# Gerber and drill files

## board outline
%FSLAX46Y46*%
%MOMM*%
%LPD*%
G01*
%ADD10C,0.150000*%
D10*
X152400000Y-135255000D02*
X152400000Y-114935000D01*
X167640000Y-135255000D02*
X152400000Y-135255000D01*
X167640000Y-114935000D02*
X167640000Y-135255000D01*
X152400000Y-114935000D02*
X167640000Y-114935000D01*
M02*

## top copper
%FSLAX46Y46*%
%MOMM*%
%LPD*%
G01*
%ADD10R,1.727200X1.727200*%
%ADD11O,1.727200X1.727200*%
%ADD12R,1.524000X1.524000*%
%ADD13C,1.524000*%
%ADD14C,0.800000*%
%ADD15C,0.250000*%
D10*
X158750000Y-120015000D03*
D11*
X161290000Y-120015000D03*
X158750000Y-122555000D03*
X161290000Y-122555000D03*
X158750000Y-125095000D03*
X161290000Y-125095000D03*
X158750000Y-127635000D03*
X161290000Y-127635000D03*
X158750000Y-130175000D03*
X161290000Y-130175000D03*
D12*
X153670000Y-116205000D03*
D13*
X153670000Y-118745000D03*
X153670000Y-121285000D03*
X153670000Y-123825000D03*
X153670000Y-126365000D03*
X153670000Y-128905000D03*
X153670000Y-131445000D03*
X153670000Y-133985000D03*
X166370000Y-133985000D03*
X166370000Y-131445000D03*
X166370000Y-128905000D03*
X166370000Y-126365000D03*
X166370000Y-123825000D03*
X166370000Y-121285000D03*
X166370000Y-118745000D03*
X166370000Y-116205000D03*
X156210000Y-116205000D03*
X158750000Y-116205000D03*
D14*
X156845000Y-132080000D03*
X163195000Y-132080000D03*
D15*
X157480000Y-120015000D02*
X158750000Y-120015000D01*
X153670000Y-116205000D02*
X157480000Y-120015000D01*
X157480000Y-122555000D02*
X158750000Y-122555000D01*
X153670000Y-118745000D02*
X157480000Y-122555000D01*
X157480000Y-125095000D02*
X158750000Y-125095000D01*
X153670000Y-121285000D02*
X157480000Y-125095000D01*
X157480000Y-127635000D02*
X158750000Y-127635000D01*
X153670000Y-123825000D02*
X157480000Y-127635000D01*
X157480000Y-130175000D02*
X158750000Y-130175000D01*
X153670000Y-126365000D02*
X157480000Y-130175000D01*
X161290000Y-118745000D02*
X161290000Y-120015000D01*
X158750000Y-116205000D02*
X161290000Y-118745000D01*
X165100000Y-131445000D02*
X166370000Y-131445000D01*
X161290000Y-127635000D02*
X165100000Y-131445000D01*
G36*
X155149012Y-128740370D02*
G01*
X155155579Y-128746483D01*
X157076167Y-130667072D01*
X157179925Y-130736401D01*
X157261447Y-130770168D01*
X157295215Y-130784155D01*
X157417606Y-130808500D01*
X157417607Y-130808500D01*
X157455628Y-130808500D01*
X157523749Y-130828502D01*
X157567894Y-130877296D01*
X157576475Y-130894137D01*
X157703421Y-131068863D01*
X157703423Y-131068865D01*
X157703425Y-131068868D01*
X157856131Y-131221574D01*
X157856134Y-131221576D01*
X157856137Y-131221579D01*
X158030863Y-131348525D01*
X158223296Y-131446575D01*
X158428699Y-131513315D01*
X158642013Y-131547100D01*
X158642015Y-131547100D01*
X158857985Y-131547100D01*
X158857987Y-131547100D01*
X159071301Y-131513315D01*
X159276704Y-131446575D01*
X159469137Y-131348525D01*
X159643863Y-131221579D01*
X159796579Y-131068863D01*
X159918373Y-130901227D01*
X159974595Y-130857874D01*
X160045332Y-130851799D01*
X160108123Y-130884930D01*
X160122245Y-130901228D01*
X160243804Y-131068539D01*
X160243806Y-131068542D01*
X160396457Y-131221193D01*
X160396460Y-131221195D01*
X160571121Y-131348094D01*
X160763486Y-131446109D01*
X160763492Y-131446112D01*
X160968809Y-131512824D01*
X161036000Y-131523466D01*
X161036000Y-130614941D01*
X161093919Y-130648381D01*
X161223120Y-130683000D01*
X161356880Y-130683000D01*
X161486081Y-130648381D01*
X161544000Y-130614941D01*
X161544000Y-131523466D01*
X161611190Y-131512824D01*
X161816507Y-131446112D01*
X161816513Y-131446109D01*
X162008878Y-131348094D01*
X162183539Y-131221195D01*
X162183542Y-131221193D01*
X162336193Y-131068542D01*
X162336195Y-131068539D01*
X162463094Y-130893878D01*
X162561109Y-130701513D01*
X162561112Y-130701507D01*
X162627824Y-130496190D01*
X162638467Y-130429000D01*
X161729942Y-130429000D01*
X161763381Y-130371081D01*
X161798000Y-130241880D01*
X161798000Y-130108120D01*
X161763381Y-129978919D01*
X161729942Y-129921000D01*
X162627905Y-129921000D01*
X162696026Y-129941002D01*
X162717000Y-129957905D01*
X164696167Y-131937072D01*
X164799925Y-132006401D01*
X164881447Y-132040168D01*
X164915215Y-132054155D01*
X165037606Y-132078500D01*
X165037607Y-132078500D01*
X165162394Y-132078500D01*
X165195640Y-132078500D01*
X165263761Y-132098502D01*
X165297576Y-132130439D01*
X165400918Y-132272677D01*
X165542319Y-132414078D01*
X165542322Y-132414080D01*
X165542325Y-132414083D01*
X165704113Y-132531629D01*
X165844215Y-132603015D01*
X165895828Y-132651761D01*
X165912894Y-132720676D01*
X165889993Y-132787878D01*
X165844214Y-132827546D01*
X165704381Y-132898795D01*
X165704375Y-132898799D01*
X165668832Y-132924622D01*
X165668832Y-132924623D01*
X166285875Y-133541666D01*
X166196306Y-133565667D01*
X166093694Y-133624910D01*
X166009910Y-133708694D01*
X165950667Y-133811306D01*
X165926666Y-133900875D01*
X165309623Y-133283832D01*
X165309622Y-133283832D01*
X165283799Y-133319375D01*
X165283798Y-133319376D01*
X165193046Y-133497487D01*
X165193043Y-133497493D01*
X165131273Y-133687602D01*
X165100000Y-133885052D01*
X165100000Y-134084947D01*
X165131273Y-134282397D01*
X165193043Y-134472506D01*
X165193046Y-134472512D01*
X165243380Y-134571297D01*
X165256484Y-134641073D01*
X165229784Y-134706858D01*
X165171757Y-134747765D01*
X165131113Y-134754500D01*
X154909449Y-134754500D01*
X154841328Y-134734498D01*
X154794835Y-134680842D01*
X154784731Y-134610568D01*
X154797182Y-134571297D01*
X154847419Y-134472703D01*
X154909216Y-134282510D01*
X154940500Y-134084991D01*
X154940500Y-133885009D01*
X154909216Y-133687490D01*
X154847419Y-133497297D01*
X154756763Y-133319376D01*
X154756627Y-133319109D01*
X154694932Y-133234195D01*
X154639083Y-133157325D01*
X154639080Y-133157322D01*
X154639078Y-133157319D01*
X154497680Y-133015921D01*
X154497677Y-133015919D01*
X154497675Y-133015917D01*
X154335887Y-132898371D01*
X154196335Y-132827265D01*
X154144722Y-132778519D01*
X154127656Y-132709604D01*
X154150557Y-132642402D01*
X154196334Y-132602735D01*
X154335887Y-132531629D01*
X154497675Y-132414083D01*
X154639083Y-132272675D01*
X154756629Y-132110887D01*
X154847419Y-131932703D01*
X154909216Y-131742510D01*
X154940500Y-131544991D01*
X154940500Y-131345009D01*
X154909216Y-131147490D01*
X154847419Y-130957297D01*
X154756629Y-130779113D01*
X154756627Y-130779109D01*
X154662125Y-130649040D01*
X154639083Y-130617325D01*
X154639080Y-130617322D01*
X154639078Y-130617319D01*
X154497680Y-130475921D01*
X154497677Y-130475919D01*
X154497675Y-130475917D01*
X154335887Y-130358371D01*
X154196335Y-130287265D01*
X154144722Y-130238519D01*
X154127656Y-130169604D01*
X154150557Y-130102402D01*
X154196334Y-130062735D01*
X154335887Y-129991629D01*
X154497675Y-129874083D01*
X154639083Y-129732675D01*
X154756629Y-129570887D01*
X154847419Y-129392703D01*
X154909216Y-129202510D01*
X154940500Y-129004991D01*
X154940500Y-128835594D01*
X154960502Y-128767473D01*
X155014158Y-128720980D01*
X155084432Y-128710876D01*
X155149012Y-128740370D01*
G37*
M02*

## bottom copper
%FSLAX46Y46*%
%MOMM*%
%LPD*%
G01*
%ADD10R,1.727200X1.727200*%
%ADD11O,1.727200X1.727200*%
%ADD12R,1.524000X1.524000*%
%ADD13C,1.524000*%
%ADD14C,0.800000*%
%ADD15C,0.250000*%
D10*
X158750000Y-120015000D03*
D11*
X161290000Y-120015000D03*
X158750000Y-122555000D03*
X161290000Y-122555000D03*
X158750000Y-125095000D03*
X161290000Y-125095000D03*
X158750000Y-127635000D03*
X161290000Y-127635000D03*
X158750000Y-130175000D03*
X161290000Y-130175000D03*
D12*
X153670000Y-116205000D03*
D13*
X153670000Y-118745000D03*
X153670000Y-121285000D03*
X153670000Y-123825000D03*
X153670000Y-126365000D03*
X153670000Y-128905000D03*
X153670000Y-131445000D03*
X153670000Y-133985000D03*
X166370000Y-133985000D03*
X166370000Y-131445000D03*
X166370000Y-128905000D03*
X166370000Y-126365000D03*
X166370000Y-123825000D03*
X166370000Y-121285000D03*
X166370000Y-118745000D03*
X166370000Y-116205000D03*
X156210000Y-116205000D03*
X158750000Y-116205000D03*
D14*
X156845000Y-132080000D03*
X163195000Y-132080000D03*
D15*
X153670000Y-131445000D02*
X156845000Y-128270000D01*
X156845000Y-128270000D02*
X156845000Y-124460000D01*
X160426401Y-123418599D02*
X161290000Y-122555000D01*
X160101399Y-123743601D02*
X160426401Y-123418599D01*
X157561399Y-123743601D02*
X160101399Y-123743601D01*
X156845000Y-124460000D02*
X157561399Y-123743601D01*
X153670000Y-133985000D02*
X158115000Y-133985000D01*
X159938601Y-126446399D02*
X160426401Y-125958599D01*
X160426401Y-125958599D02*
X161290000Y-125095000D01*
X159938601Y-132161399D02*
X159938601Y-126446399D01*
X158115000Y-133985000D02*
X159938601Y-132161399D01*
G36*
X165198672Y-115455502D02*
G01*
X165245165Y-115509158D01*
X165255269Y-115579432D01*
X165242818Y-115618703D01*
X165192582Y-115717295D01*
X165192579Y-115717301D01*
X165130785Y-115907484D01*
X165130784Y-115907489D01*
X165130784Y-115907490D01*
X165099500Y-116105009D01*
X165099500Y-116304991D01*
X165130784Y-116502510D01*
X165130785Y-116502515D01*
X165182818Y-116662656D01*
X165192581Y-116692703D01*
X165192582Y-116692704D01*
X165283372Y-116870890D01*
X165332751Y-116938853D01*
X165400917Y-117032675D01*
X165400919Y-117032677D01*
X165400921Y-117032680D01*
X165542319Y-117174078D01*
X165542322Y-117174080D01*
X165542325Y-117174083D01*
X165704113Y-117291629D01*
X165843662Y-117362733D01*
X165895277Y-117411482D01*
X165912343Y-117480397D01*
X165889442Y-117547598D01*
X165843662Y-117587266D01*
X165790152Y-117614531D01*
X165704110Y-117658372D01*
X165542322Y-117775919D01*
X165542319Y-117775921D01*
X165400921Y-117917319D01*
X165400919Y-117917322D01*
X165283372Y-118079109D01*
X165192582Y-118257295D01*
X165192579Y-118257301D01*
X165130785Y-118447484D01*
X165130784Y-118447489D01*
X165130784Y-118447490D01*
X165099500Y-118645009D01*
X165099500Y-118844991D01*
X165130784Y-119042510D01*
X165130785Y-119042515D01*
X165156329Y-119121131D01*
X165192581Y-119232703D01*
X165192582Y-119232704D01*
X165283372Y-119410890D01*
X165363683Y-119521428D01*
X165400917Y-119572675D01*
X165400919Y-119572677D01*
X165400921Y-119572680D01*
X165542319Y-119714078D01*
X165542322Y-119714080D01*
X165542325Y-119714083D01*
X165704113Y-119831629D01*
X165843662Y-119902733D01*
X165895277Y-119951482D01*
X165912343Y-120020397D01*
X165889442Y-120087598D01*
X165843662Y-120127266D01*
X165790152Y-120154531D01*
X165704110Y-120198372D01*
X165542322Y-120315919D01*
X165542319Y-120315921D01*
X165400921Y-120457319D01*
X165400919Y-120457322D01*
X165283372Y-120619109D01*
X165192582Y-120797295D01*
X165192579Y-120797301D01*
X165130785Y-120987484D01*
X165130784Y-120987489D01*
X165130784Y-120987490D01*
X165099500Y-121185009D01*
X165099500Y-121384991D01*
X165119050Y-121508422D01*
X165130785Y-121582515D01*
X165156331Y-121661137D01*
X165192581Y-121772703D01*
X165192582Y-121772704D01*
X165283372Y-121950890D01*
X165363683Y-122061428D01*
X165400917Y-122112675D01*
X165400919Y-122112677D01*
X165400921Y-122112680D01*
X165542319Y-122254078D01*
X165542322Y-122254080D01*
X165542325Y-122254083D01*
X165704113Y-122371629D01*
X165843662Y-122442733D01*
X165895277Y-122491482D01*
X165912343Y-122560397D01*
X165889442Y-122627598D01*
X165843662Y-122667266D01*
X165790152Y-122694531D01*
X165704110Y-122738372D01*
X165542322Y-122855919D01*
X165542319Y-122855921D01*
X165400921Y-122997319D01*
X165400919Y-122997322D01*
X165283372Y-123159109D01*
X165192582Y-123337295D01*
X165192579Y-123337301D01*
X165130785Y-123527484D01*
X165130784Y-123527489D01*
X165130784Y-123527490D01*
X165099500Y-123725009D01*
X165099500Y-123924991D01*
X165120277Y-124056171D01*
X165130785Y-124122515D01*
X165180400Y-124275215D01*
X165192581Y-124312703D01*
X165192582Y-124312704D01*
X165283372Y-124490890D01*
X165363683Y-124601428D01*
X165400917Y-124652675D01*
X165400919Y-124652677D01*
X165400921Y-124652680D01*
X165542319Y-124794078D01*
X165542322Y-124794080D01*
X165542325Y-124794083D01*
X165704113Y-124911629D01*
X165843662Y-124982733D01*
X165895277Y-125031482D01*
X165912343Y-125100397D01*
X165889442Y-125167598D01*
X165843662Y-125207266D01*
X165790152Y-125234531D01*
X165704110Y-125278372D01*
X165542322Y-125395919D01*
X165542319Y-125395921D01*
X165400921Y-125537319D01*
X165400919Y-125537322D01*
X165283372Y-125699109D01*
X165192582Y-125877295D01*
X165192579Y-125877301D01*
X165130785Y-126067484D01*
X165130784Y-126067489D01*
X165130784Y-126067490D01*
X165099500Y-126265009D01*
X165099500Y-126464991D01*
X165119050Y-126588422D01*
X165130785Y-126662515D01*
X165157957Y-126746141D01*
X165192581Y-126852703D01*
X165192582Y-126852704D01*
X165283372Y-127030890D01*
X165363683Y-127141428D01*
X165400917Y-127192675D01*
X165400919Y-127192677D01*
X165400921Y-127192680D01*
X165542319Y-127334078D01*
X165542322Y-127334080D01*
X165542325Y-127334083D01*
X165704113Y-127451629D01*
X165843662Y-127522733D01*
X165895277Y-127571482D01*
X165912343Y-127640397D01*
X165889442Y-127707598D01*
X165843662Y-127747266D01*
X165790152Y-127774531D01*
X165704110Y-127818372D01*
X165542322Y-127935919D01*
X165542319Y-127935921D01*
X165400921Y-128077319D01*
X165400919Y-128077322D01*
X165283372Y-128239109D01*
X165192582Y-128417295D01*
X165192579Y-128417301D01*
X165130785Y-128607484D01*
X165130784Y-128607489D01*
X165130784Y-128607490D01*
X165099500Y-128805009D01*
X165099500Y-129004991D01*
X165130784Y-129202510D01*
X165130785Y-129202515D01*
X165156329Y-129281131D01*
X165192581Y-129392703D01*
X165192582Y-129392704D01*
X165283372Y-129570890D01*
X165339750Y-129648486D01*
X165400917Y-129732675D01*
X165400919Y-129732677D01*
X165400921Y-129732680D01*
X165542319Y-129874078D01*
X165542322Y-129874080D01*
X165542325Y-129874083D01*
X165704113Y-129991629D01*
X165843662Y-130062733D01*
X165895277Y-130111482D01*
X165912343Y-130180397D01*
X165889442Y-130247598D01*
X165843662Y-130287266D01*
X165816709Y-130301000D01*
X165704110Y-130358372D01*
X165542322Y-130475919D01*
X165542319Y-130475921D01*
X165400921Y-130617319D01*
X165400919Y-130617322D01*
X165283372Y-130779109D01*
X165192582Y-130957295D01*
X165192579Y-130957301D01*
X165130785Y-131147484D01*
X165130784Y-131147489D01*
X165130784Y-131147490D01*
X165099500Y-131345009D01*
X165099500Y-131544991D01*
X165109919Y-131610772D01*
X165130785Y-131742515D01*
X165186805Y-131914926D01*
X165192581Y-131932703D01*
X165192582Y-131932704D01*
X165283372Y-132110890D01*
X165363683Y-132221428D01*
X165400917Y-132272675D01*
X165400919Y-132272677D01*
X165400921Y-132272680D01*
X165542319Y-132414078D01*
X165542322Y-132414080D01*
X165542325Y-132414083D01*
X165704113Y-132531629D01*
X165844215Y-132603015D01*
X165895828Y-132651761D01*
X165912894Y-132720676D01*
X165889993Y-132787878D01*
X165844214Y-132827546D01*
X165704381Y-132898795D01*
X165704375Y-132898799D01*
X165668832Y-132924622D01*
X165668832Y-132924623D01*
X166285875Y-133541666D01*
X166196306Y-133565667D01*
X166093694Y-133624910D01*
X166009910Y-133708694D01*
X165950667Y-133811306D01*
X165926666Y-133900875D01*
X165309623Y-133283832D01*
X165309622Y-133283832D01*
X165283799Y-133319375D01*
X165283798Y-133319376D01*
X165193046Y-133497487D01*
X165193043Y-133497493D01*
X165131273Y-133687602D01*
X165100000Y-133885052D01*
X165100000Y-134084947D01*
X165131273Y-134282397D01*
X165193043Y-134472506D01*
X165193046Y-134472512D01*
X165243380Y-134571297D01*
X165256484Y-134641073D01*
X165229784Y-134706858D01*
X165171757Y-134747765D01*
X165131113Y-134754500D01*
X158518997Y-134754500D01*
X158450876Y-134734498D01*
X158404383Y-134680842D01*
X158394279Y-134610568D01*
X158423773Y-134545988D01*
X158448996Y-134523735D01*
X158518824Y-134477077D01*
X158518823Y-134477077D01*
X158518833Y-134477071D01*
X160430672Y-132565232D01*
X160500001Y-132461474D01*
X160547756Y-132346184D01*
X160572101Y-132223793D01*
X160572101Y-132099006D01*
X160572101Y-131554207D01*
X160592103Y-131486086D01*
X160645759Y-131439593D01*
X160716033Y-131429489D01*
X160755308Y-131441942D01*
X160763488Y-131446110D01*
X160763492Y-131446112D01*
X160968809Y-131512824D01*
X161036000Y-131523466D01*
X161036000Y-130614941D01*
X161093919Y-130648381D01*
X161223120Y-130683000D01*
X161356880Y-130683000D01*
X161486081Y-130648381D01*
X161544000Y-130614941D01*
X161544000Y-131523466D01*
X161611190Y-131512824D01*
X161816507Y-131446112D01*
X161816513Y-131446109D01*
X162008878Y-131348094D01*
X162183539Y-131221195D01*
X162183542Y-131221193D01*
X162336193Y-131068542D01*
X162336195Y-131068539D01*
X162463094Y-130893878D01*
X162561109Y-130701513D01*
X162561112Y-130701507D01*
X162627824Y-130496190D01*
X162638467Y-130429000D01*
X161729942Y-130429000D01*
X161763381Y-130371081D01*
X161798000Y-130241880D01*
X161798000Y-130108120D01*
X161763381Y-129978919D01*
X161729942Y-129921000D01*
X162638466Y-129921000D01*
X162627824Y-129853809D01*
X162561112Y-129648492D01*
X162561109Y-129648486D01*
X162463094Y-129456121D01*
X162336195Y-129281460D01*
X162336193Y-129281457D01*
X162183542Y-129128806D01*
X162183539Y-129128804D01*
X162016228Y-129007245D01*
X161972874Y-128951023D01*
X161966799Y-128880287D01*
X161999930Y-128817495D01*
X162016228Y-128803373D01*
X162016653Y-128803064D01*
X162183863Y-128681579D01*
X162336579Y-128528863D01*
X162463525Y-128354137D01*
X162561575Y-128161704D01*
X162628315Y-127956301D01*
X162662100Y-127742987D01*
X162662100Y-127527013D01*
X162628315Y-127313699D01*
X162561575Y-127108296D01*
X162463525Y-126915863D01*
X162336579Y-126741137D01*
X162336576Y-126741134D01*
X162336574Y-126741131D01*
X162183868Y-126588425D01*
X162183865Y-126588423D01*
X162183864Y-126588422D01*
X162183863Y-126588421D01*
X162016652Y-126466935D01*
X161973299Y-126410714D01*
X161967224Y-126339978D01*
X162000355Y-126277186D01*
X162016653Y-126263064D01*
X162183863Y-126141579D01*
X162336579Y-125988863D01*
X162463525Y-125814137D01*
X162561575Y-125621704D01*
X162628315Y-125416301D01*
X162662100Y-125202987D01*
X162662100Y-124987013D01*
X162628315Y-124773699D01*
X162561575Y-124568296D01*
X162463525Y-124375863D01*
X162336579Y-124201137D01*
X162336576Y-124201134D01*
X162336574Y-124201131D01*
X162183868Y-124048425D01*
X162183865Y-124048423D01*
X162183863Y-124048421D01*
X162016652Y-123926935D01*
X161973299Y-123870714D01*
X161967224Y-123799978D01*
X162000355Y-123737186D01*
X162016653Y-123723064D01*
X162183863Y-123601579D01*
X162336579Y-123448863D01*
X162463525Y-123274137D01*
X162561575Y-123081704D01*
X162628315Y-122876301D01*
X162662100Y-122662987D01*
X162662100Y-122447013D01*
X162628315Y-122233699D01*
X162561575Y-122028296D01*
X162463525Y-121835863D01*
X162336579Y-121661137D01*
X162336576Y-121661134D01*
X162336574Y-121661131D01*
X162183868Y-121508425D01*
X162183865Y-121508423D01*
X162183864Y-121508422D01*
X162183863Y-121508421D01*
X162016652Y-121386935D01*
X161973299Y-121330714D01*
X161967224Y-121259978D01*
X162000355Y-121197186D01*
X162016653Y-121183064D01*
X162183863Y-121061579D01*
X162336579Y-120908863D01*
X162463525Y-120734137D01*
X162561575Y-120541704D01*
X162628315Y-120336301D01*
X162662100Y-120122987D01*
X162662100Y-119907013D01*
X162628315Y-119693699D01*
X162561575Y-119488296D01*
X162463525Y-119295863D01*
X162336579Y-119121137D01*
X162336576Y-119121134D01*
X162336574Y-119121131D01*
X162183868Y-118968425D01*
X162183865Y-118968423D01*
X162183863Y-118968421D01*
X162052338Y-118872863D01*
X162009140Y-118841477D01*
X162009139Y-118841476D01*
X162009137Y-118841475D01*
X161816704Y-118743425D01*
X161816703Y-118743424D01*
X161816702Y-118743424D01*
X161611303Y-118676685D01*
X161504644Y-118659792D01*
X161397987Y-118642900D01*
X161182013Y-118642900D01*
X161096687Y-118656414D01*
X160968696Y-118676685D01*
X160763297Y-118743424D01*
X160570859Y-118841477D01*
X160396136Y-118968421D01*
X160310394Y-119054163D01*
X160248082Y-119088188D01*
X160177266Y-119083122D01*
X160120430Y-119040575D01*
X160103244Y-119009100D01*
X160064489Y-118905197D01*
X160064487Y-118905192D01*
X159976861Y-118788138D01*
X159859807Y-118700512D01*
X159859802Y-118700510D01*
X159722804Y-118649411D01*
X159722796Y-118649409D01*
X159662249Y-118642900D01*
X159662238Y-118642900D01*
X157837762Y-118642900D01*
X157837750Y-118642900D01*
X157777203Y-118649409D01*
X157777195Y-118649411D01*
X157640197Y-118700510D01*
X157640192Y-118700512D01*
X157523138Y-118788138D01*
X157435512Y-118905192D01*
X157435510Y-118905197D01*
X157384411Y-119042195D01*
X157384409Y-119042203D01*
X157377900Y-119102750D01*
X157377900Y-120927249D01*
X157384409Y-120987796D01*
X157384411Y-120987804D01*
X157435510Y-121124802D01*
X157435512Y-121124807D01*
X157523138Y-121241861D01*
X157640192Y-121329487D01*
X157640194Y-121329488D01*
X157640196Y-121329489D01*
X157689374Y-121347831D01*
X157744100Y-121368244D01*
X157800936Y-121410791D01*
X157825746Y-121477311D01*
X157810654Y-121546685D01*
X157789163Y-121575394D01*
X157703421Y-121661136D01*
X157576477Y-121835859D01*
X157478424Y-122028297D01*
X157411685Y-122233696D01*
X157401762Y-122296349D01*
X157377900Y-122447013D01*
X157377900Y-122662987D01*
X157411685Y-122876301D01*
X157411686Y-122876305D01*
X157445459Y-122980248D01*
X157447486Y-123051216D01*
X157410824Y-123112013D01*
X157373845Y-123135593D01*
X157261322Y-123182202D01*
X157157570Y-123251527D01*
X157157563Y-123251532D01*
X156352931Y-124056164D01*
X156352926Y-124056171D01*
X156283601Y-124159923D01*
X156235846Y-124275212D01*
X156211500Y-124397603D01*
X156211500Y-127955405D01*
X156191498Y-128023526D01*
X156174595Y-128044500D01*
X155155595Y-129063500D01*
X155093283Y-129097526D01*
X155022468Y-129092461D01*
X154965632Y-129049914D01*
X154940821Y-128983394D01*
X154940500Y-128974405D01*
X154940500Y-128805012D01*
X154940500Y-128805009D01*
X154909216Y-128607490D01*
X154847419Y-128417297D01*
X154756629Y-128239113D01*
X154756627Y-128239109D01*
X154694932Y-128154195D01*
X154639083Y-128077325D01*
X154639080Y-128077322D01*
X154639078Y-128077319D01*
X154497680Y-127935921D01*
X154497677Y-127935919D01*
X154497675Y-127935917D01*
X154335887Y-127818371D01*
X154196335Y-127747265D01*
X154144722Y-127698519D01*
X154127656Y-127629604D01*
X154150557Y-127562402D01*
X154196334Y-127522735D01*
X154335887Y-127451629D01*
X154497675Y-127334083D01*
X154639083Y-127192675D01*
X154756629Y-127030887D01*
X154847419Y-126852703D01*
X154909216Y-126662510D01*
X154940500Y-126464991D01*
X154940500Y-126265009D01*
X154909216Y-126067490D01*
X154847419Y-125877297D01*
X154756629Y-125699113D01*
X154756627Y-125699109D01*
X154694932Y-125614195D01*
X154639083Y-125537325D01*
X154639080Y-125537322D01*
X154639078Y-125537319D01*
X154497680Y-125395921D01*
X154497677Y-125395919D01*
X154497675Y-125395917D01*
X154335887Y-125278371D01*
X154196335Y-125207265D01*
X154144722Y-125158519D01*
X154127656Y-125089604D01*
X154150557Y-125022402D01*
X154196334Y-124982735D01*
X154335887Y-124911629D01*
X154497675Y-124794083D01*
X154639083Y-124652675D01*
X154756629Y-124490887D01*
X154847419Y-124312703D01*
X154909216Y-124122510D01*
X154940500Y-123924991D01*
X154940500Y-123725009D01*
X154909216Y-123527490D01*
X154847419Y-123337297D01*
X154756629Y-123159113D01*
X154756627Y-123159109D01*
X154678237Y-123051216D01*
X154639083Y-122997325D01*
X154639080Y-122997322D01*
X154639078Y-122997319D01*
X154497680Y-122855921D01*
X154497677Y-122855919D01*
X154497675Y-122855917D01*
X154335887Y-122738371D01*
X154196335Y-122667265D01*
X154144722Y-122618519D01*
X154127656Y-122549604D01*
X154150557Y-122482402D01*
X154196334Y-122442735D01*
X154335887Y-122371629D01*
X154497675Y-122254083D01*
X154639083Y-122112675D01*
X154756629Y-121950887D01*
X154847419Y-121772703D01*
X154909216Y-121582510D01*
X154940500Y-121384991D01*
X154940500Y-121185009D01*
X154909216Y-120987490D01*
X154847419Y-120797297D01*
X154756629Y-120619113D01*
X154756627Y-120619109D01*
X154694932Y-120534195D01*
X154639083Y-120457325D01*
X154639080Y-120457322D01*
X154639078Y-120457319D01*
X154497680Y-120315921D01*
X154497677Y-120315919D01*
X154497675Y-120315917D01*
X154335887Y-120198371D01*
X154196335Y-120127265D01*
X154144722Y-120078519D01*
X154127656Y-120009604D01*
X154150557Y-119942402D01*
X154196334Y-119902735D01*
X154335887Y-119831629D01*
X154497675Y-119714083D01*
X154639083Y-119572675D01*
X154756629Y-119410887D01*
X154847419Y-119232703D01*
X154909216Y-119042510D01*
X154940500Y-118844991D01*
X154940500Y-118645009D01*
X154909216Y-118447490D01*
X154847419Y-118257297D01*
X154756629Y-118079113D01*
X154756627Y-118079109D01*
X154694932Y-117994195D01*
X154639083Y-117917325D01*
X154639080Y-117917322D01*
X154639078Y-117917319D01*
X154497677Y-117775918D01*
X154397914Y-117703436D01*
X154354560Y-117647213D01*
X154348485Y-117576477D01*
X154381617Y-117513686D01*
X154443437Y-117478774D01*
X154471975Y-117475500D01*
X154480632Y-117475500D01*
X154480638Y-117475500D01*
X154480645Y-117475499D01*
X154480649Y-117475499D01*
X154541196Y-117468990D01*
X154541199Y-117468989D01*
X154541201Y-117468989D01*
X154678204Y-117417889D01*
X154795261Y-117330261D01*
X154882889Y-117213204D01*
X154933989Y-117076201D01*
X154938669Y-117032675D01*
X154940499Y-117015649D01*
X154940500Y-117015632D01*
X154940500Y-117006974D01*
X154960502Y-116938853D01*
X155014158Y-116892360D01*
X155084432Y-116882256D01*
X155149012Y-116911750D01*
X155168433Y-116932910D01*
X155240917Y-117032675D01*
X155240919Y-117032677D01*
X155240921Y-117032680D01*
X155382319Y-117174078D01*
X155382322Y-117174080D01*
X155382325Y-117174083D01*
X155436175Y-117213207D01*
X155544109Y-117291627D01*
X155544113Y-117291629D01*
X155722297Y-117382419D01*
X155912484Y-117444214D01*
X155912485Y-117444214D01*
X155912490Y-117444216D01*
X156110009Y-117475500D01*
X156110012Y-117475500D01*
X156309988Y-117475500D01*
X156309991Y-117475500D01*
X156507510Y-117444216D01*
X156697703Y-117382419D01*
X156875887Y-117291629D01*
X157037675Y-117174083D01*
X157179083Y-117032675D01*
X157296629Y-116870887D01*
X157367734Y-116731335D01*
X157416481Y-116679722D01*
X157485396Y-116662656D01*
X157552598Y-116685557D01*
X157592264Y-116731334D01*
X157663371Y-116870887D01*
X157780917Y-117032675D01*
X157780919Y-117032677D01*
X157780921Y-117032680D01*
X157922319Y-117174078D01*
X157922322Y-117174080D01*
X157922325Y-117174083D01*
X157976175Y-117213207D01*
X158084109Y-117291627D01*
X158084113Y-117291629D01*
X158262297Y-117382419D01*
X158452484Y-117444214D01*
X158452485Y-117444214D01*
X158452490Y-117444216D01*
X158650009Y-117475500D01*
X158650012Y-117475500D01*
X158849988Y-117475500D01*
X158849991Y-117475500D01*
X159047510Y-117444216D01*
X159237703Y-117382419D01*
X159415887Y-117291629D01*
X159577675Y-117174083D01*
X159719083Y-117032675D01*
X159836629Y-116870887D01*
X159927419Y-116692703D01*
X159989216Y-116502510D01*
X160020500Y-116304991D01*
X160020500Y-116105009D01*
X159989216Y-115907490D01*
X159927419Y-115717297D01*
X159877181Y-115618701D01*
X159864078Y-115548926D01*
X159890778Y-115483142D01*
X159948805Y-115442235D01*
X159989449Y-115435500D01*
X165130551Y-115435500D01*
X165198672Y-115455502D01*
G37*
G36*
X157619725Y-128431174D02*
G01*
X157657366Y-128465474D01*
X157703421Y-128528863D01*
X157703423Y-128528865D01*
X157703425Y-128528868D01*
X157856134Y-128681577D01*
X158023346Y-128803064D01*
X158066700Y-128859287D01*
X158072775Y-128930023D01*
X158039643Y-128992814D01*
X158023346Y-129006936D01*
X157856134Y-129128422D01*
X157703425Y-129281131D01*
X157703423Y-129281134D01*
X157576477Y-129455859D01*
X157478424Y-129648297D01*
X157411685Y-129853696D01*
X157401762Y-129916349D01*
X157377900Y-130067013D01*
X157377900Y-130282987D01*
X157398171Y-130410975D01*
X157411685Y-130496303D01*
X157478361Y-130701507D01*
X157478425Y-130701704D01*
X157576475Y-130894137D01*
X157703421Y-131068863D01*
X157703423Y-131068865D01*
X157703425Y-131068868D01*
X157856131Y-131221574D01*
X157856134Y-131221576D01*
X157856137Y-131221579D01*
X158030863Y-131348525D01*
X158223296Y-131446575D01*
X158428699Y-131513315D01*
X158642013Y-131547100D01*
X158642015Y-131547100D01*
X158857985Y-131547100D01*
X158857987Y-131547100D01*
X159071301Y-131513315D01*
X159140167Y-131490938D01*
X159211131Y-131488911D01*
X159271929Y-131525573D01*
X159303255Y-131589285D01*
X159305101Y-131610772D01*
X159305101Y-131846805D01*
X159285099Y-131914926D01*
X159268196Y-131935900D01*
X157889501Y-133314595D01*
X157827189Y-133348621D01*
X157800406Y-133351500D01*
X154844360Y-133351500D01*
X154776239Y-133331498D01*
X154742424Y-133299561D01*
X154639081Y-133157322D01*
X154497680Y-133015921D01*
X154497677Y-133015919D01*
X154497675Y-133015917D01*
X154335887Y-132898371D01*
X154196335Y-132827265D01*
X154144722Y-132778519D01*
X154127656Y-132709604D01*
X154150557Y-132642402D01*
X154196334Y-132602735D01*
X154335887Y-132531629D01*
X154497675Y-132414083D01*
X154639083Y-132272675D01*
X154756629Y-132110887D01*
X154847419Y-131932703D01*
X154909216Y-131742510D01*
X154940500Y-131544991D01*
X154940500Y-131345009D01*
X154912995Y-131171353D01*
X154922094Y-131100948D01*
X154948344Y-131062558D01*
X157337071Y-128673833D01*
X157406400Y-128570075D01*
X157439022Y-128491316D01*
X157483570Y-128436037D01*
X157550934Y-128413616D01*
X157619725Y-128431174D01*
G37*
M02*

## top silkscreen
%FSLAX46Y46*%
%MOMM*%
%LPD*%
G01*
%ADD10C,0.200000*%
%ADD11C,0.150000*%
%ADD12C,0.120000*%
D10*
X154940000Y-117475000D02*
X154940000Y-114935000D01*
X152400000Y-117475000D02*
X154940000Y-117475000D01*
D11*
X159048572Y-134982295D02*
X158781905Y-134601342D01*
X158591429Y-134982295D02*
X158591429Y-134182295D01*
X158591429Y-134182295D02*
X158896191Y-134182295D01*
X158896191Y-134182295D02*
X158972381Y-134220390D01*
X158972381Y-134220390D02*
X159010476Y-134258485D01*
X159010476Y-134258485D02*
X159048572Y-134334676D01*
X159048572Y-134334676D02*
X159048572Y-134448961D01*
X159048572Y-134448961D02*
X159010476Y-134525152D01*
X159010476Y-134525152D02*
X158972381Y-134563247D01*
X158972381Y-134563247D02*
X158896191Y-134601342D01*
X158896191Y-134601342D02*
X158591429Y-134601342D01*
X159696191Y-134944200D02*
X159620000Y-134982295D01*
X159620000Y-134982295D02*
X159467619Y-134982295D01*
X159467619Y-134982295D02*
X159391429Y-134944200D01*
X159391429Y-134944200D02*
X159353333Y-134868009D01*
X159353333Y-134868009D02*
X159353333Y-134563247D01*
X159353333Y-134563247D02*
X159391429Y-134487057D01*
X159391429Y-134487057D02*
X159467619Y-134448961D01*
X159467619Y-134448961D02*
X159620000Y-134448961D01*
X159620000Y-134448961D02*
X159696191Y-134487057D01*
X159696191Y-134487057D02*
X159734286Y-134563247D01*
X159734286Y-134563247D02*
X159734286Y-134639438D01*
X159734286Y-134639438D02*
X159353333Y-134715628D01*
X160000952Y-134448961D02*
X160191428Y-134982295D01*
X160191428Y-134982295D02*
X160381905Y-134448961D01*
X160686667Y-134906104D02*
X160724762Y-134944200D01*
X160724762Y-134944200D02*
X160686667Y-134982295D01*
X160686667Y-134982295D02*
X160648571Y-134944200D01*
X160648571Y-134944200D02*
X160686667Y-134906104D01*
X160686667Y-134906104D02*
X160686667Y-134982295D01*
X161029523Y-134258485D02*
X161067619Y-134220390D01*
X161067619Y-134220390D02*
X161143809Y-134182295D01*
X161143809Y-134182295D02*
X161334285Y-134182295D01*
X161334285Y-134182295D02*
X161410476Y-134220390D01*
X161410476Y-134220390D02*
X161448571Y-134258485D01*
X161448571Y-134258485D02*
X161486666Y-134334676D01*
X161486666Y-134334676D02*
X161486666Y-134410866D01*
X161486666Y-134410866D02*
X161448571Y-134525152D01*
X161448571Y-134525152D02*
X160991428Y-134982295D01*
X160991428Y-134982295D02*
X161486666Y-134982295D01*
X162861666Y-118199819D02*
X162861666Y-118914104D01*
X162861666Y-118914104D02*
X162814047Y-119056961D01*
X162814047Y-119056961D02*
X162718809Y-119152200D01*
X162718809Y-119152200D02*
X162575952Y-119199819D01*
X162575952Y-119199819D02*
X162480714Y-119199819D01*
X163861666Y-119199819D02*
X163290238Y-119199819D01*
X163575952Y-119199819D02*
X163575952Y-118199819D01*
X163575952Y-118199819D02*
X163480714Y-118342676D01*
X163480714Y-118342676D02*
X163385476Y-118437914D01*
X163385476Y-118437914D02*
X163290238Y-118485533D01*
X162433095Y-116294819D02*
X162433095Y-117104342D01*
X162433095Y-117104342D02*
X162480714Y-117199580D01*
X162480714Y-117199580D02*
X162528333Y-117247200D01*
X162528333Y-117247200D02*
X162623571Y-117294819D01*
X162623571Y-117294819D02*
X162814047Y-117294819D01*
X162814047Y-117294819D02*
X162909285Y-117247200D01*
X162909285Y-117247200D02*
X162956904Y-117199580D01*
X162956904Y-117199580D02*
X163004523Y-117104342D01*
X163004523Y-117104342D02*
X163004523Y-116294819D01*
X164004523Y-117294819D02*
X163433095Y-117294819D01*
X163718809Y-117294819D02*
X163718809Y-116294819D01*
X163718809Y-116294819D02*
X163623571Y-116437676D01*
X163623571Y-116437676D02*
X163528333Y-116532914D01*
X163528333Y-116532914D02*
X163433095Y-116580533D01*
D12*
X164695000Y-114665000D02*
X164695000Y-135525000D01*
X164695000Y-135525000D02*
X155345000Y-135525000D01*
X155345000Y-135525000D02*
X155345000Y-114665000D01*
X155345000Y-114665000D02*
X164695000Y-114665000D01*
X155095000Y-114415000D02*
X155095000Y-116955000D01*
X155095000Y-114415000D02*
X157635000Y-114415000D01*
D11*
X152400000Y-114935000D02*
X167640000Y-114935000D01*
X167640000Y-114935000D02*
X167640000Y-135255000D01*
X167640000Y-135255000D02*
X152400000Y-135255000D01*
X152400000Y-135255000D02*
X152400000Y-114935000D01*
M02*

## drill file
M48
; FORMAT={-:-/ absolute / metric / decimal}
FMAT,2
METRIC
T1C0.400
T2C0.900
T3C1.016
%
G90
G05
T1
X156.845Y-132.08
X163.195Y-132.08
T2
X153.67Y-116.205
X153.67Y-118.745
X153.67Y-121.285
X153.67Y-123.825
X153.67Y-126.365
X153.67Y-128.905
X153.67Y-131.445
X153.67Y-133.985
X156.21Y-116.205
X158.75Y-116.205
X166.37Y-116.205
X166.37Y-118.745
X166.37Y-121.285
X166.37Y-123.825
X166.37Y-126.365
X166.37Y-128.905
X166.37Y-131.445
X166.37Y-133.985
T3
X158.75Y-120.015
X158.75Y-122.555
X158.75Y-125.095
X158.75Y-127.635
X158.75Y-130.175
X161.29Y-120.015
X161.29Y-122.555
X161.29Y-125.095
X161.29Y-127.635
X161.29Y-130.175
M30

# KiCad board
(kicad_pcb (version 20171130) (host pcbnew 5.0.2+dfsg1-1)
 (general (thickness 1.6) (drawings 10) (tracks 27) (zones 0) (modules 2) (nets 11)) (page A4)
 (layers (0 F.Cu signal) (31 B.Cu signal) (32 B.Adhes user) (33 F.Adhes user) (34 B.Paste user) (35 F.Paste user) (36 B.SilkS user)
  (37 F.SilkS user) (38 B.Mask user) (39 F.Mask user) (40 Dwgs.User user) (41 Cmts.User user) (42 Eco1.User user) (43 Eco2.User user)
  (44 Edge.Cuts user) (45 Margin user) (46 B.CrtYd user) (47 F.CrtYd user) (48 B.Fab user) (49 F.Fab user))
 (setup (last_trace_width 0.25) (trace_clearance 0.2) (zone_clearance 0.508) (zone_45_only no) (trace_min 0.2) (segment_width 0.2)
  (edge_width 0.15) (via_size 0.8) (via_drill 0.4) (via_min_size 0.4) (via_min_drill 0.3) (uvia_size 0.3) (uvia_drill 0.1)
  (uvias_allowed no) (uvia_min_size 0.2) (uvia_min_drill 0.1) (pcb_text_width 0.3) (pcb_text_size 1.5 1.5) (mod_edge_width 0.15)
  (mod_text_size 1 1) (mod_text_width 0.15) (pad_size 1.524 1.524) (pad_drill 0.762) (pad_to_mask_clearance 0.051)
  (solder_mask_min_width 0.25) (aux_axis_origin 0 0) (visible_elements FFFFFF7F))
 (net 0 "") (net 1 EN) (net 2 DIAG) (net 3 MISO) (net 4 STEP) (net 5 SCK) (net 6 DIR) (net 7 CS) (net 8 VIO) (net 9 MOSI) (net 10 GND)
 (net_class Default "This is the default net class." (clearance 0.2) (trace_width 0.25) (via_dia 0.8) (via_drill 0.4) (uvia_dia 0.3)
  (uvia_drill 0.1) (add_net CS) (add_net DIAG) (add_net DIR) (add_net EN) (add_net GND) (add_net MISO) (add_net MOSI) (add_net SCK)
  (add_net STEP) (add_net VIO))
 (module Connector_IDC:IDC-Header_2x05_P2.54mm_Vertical (layer F.Cu) (at 158.75 120.015)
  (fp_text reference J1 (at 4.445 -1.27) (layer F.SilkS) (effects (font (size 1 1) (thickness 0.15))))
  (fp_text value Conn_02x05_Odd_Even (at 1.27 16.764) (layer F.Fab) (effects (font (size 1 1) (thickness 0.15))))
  (fp_line (start 5.945 -5.35) (end 5.945 15.51) (layer F.SilkS) (width 0.12))
  (fp_line (start 5.945 15.51) (end -3.405 15.51) (layer F.SilkS) (width 0.12))
  (fp_line (start -3.405 15.51) (end -3.405 -5.35) (layer F.SilkS) (width 0.12))
  (fp_line (start -3.405 -5.35) (end 5.945 -5.35) (layer F.SilkS) (width 0.12))
  (fp_line (start -3.655 -5.6) (end -3.655 -3.06) (layer F.SilkS) (width 0.12))
  (fp_line (start -3.655 -5.6) (end -1.115 -5.6) (layer F.SilkS) (width 0.12))
  (pad 1 thru_hole rect (at 0 0) (size 1.7272 1.7272) (drill 1.016) (layers *.Cu *.Mask) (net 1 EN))
  (pad 2 thru_hole oval (at 2.54 0) (size 1.7272 1.7272) (drill 1.016) (layers *.Cu *.Mask) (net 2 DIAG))
  (pad 3 thru_hole oval (at 0 2.54) (size 1.7272 1.7272) (drill 1.016) (layers *.Cu *.Mask) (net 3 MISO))
  (pad 4 thru_hole oval (at 2.54 2.54) (size 1.7272 1.7272) (drill 1.016) (layers *.Cu *.Mask) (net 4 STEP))
  (pad 5 thru_hole oval (at 0 5.08) (size 1.7272 1.7272) (drill 1.016) (layers *.Cu *.Mask) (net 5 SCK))
  (pad 6 thru_hole oval (at 2.54 5.08) (size 1.7272 1.7272) (drill 1.016) (layers *.Cu *.Mask) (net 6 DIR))
  (pad 7 thru_hole oval (at 0 7.62) (size 1.7272 1.7272) (drill 1.016) (layers *.Cu *.Mask) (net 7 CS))
  (pad 8 thru_hole oval (at 2.54 7.62) (size 1.7272 1.7272) (drill 1.016) (layers *.Cu *.Mask) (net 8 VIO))
  (pad 9 thru_hole oval (at 0 10.16) (size 1.7272 1.7272) (drill 1.016) (layers *.Cu *.Mask) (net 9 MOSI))
  (pad 10 thru_hole oval (at 2.54 10.16) (size 1.7272 1.7272) (drill 1.016) (layers *.Cu *.Mask) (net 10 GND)))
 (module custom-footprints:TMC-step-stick (layer F.Cu) (at 158.75 133.985)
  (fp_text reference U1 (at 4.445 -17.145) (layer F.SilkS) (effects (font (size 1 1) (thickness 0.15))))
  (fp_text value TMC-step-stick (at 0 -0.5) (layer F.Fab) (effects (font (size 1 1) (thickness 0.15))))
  (fp_line (start -6.35 -19.05) (end 8.89 -19.05) (layer F.SilkS) (width 0.15))
  (fp_line (start 8.89 -19.05) (end 8.89 1.27) (layer F.SilkS) (width 0.15))
  (fp_line (start 8.89 1.27) (end -6.35 1.27) (layer F.SilkS) (width 0.15))
  (fp_line (start -6.35 1.27) (end -6.35 -19.05) (layer F.SilkS) (width 0.15))
  (pad 1 thru_hole rect (at -5.08 -17.78) (size 1.524 1.524) (drill 0.9) (layers *.Cu *.Mask) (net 1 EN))
  (pad 2 thru_hole circle (at -5.08 -15.24) (size 1.524 1.524) (drill 0.9) (layers *.Cu *.Mask) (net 3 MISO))
  (pad 3 thru_hole circle (at -5.08 -12.7) (size 1.524 1.524) (drill 0.9) (layers *.Cu *.Mask) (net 5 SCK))
  (pad 4 thru_hole circle (at -5.08 -10.16) (size 1.524 1.524) (drill 0.9) (layers *.Cu *.Mask) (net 7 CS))
  (pad 5 thru_hole circle (at -5.08 -7.62) (size 1.524 1.524) (drill 0.9) (layers *.Cu *.Mask) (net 9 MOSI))
  (pad 6 thru_hole circle (at -5.08 -5.08) (size 1.524 1.524) (drill 0.9) (layers *.Cu *.Mask))
  (pad 7 thru_hole circle (at -5.08 -2.54) (size 1.524 1.524) (drill 0.9) (layers *.Cu *.Mask) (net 4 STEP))
  (pad 8 thru_hole circle (at -5.08 0) (size 1.524 1.524) (drill 0.9) (layers *.Cu *.Mask) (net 6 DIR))
  (pad 9 thru_hole circle (at 7.62 0) (size 1.524 1.524) (drill 0.9) (layers *.Cu *.Mask) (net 10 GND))
  (pad 10 thru_hole circle (at 7.62 -2.54) (size 1.524 1.524) (drill 0.9) (layers *.Cu *.Mask) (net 8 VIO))
  (pad 11 thru_hole circle (at 7.62 -5.08) (size 1.524 1.524) (drill 0.9) (layers *.Cu *.Mask))
  (pad 12 thru_hole circle (at 7.62 -7.62) (size 1.524 1.524) (drill 0.9) (layers *.Cu *.Mask))
  (pad 13 thru_hole circle (at 7.62 -10.16) (size 1.524 1.524) (drill 0.9) (layers *.Cu *.Mask))
  (pad 14 thru_hole circle (at 7.62 -12.7) (size 1.524 1.524) (drill 0.9) (layers *.Cu *.Mask))
  (pad 15 thru_hole circle (at 7.62 -15.24) (size 1.524 1.524) (drill 0.9) (layers *.Cu *.Mask))
  (pad 16 thru_hole circle (at 7.62 -17.78) (size 1.524 1.524) (drill 0.9) (layers *.Cu *.Mask))
  (pad 17 thru_hole circle (at -2.54 -17.78) (size 1.524 1.524) (drill 0.9) (layers *.Cu *.Mask))
  (pad 18 thru_hole circle (at 0 -17.78) (size 1.524 1.524) (drill 0.9) (layers *.Cu *.Mask) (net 2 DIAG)))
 (gr_line (start 154.94 117.475) (end 154.94 114.935) (layer F.SilkS) (width 0.2))
 (gr_line (start 152.4 117.475) (end 154.94 117.475) (layer F.SilkS) (width 0.2))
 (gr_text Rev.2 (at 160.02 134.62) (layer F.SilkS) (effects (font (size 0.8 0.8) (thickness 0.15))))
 (gr_line (start 152.4 135.255) (end 152.4 114.935) (layer Edge.Cuts) (width 0.15))
 (gr_line (start 167.64 135.255) (end 152.4 135.255) (layer Edge.Cuts) (width 0.15))
 (gr_line (start 167.64 114.935) (end 167.64 135.255) (layer Edge.Cuts) (width 0.15))
 (gr_line (start 152.4 114.935) (end 167.64 114.935) (layer Edge.Cuts) (width 0.15))
 (segment (start 157.48 120.015) (end 158.75 120.015) (width 0.25) (layer F.Cu) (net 1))
 (segment (start 153.67 116.205) (end 157.48 120.015) (width 0.25) (layer F.Cu) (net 1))
 (segment (start 157.48 122.555) (end 158.75 122.555) (width 0.25) (layer F.Cu) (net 3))
 (segment (start 153.67 118.745) (end 157.48 122.555) (width 0.25) (layer F.Cu) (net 3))
 (segment (start 157.48 125.095) (end 158.75 125.095) (width 0.25) (layer F.Cu) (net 5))
 (segment (start 153.67 121.285) (end 157.48 125.095) (width 0.25) (layer F.Cu) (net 5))
 (segment (start 157.48 127.635) (end 158.75 127.635) (width 0.25) (layer F.Cu) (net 7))
 (segment (start 153.67 123.825) (end 157.48 127.635) (width 0.25) (layer F.Cu) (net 7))
 (segment (start 157.48 130.175) (end 158.75 130.175) (width 0.25) (layer F.Cu) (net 9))
 (segment (start 153.67 126.365) (end 157.48 130.175) (width 0.25) (layer F.Cu) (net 9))
 (segment (start 161.29 118.745) (end 161.29 120.015) (width 0.25) (layer F.Cu) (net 2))
 (segment (start 158.75 116.205) (end 161.29 118.745) (width 0.25) (layer F.Cu) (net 2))
 (segment (start 153.67 131.445) (end 156.845 128.27) (width 0.25) (layer B.Cu) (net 4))
 (segment (start 156.845 128.27) (end 156.845 124.46) (width 0.25) (layer B.Cu) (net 4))
 (segment (start 160.426401 123.418599) (end 161.29 122.555) (width 0.25) (layer B.Cu) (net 4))
 (segment (start 160.101399 123.743601) (end 160.426401 123.418599) (width 0.25) (layer B.Cu) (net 4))
 (segment (start 157.561399 123.743601) (end 160.101399 123.743601) (width 0.25) (layer B.Cu) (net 4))
 (segment (start 156.845 124.46) (end 157.561399 123.743601) (width 0.25) (layer B.Cu) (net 4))
 (segment (start 153.67 133.985) (end 158.115 133.985) (width 0.25) (layer B.Cu) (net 6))
 (segment (start 159.938601 126.446399) (end 160.426401 125.958599) (width 0.25) (layer B.Cu) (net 6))
 (segment (start 160.426401 125.958599) (end 161.29 125.095) (width 0.25) (layer B.Cu) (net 6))
 (segment (start 159.938601 132.161399) (end 159.938601 126.446399) (width 0.25) (layer B.Cu) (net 6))
 (segment (start 158.115 133.985) (end 159.938601 132.161399) (width 0.25) (layer B.Cu) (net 6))
 (segment (start 165.1 131.445) (end 166.37 131.445) (width 0.25) (layer F.Cu) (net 8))
 (segment (start 161.29 127.635) (end 165.1 131.445) (width 0.25) (layer F.Cu) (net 8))
 (via (at 156.845 132.08) (size 0.8) (drill 0.4) (layers F.Cu B.Cu) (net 10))
 (via (at 163.195 132.08) (size 0.8) (drill 0.4) (layers F.Cu B.Cu) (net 10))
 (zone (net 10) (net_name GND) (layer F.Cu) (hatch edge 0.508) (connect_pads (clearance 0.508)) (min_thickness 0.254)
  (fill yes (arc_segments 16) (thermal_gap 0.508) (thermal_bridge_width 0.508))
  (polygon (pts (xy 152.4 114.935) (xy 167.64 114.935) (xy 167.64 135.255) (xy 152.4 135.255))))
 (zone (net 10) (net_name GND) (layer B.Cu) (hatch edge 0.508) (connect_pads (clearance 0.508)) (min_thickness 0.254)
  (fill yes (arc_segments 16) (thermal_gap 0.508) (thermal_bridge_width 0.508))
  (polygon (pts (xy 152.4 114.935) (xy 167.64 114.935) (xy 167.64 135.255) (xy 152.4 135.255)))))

